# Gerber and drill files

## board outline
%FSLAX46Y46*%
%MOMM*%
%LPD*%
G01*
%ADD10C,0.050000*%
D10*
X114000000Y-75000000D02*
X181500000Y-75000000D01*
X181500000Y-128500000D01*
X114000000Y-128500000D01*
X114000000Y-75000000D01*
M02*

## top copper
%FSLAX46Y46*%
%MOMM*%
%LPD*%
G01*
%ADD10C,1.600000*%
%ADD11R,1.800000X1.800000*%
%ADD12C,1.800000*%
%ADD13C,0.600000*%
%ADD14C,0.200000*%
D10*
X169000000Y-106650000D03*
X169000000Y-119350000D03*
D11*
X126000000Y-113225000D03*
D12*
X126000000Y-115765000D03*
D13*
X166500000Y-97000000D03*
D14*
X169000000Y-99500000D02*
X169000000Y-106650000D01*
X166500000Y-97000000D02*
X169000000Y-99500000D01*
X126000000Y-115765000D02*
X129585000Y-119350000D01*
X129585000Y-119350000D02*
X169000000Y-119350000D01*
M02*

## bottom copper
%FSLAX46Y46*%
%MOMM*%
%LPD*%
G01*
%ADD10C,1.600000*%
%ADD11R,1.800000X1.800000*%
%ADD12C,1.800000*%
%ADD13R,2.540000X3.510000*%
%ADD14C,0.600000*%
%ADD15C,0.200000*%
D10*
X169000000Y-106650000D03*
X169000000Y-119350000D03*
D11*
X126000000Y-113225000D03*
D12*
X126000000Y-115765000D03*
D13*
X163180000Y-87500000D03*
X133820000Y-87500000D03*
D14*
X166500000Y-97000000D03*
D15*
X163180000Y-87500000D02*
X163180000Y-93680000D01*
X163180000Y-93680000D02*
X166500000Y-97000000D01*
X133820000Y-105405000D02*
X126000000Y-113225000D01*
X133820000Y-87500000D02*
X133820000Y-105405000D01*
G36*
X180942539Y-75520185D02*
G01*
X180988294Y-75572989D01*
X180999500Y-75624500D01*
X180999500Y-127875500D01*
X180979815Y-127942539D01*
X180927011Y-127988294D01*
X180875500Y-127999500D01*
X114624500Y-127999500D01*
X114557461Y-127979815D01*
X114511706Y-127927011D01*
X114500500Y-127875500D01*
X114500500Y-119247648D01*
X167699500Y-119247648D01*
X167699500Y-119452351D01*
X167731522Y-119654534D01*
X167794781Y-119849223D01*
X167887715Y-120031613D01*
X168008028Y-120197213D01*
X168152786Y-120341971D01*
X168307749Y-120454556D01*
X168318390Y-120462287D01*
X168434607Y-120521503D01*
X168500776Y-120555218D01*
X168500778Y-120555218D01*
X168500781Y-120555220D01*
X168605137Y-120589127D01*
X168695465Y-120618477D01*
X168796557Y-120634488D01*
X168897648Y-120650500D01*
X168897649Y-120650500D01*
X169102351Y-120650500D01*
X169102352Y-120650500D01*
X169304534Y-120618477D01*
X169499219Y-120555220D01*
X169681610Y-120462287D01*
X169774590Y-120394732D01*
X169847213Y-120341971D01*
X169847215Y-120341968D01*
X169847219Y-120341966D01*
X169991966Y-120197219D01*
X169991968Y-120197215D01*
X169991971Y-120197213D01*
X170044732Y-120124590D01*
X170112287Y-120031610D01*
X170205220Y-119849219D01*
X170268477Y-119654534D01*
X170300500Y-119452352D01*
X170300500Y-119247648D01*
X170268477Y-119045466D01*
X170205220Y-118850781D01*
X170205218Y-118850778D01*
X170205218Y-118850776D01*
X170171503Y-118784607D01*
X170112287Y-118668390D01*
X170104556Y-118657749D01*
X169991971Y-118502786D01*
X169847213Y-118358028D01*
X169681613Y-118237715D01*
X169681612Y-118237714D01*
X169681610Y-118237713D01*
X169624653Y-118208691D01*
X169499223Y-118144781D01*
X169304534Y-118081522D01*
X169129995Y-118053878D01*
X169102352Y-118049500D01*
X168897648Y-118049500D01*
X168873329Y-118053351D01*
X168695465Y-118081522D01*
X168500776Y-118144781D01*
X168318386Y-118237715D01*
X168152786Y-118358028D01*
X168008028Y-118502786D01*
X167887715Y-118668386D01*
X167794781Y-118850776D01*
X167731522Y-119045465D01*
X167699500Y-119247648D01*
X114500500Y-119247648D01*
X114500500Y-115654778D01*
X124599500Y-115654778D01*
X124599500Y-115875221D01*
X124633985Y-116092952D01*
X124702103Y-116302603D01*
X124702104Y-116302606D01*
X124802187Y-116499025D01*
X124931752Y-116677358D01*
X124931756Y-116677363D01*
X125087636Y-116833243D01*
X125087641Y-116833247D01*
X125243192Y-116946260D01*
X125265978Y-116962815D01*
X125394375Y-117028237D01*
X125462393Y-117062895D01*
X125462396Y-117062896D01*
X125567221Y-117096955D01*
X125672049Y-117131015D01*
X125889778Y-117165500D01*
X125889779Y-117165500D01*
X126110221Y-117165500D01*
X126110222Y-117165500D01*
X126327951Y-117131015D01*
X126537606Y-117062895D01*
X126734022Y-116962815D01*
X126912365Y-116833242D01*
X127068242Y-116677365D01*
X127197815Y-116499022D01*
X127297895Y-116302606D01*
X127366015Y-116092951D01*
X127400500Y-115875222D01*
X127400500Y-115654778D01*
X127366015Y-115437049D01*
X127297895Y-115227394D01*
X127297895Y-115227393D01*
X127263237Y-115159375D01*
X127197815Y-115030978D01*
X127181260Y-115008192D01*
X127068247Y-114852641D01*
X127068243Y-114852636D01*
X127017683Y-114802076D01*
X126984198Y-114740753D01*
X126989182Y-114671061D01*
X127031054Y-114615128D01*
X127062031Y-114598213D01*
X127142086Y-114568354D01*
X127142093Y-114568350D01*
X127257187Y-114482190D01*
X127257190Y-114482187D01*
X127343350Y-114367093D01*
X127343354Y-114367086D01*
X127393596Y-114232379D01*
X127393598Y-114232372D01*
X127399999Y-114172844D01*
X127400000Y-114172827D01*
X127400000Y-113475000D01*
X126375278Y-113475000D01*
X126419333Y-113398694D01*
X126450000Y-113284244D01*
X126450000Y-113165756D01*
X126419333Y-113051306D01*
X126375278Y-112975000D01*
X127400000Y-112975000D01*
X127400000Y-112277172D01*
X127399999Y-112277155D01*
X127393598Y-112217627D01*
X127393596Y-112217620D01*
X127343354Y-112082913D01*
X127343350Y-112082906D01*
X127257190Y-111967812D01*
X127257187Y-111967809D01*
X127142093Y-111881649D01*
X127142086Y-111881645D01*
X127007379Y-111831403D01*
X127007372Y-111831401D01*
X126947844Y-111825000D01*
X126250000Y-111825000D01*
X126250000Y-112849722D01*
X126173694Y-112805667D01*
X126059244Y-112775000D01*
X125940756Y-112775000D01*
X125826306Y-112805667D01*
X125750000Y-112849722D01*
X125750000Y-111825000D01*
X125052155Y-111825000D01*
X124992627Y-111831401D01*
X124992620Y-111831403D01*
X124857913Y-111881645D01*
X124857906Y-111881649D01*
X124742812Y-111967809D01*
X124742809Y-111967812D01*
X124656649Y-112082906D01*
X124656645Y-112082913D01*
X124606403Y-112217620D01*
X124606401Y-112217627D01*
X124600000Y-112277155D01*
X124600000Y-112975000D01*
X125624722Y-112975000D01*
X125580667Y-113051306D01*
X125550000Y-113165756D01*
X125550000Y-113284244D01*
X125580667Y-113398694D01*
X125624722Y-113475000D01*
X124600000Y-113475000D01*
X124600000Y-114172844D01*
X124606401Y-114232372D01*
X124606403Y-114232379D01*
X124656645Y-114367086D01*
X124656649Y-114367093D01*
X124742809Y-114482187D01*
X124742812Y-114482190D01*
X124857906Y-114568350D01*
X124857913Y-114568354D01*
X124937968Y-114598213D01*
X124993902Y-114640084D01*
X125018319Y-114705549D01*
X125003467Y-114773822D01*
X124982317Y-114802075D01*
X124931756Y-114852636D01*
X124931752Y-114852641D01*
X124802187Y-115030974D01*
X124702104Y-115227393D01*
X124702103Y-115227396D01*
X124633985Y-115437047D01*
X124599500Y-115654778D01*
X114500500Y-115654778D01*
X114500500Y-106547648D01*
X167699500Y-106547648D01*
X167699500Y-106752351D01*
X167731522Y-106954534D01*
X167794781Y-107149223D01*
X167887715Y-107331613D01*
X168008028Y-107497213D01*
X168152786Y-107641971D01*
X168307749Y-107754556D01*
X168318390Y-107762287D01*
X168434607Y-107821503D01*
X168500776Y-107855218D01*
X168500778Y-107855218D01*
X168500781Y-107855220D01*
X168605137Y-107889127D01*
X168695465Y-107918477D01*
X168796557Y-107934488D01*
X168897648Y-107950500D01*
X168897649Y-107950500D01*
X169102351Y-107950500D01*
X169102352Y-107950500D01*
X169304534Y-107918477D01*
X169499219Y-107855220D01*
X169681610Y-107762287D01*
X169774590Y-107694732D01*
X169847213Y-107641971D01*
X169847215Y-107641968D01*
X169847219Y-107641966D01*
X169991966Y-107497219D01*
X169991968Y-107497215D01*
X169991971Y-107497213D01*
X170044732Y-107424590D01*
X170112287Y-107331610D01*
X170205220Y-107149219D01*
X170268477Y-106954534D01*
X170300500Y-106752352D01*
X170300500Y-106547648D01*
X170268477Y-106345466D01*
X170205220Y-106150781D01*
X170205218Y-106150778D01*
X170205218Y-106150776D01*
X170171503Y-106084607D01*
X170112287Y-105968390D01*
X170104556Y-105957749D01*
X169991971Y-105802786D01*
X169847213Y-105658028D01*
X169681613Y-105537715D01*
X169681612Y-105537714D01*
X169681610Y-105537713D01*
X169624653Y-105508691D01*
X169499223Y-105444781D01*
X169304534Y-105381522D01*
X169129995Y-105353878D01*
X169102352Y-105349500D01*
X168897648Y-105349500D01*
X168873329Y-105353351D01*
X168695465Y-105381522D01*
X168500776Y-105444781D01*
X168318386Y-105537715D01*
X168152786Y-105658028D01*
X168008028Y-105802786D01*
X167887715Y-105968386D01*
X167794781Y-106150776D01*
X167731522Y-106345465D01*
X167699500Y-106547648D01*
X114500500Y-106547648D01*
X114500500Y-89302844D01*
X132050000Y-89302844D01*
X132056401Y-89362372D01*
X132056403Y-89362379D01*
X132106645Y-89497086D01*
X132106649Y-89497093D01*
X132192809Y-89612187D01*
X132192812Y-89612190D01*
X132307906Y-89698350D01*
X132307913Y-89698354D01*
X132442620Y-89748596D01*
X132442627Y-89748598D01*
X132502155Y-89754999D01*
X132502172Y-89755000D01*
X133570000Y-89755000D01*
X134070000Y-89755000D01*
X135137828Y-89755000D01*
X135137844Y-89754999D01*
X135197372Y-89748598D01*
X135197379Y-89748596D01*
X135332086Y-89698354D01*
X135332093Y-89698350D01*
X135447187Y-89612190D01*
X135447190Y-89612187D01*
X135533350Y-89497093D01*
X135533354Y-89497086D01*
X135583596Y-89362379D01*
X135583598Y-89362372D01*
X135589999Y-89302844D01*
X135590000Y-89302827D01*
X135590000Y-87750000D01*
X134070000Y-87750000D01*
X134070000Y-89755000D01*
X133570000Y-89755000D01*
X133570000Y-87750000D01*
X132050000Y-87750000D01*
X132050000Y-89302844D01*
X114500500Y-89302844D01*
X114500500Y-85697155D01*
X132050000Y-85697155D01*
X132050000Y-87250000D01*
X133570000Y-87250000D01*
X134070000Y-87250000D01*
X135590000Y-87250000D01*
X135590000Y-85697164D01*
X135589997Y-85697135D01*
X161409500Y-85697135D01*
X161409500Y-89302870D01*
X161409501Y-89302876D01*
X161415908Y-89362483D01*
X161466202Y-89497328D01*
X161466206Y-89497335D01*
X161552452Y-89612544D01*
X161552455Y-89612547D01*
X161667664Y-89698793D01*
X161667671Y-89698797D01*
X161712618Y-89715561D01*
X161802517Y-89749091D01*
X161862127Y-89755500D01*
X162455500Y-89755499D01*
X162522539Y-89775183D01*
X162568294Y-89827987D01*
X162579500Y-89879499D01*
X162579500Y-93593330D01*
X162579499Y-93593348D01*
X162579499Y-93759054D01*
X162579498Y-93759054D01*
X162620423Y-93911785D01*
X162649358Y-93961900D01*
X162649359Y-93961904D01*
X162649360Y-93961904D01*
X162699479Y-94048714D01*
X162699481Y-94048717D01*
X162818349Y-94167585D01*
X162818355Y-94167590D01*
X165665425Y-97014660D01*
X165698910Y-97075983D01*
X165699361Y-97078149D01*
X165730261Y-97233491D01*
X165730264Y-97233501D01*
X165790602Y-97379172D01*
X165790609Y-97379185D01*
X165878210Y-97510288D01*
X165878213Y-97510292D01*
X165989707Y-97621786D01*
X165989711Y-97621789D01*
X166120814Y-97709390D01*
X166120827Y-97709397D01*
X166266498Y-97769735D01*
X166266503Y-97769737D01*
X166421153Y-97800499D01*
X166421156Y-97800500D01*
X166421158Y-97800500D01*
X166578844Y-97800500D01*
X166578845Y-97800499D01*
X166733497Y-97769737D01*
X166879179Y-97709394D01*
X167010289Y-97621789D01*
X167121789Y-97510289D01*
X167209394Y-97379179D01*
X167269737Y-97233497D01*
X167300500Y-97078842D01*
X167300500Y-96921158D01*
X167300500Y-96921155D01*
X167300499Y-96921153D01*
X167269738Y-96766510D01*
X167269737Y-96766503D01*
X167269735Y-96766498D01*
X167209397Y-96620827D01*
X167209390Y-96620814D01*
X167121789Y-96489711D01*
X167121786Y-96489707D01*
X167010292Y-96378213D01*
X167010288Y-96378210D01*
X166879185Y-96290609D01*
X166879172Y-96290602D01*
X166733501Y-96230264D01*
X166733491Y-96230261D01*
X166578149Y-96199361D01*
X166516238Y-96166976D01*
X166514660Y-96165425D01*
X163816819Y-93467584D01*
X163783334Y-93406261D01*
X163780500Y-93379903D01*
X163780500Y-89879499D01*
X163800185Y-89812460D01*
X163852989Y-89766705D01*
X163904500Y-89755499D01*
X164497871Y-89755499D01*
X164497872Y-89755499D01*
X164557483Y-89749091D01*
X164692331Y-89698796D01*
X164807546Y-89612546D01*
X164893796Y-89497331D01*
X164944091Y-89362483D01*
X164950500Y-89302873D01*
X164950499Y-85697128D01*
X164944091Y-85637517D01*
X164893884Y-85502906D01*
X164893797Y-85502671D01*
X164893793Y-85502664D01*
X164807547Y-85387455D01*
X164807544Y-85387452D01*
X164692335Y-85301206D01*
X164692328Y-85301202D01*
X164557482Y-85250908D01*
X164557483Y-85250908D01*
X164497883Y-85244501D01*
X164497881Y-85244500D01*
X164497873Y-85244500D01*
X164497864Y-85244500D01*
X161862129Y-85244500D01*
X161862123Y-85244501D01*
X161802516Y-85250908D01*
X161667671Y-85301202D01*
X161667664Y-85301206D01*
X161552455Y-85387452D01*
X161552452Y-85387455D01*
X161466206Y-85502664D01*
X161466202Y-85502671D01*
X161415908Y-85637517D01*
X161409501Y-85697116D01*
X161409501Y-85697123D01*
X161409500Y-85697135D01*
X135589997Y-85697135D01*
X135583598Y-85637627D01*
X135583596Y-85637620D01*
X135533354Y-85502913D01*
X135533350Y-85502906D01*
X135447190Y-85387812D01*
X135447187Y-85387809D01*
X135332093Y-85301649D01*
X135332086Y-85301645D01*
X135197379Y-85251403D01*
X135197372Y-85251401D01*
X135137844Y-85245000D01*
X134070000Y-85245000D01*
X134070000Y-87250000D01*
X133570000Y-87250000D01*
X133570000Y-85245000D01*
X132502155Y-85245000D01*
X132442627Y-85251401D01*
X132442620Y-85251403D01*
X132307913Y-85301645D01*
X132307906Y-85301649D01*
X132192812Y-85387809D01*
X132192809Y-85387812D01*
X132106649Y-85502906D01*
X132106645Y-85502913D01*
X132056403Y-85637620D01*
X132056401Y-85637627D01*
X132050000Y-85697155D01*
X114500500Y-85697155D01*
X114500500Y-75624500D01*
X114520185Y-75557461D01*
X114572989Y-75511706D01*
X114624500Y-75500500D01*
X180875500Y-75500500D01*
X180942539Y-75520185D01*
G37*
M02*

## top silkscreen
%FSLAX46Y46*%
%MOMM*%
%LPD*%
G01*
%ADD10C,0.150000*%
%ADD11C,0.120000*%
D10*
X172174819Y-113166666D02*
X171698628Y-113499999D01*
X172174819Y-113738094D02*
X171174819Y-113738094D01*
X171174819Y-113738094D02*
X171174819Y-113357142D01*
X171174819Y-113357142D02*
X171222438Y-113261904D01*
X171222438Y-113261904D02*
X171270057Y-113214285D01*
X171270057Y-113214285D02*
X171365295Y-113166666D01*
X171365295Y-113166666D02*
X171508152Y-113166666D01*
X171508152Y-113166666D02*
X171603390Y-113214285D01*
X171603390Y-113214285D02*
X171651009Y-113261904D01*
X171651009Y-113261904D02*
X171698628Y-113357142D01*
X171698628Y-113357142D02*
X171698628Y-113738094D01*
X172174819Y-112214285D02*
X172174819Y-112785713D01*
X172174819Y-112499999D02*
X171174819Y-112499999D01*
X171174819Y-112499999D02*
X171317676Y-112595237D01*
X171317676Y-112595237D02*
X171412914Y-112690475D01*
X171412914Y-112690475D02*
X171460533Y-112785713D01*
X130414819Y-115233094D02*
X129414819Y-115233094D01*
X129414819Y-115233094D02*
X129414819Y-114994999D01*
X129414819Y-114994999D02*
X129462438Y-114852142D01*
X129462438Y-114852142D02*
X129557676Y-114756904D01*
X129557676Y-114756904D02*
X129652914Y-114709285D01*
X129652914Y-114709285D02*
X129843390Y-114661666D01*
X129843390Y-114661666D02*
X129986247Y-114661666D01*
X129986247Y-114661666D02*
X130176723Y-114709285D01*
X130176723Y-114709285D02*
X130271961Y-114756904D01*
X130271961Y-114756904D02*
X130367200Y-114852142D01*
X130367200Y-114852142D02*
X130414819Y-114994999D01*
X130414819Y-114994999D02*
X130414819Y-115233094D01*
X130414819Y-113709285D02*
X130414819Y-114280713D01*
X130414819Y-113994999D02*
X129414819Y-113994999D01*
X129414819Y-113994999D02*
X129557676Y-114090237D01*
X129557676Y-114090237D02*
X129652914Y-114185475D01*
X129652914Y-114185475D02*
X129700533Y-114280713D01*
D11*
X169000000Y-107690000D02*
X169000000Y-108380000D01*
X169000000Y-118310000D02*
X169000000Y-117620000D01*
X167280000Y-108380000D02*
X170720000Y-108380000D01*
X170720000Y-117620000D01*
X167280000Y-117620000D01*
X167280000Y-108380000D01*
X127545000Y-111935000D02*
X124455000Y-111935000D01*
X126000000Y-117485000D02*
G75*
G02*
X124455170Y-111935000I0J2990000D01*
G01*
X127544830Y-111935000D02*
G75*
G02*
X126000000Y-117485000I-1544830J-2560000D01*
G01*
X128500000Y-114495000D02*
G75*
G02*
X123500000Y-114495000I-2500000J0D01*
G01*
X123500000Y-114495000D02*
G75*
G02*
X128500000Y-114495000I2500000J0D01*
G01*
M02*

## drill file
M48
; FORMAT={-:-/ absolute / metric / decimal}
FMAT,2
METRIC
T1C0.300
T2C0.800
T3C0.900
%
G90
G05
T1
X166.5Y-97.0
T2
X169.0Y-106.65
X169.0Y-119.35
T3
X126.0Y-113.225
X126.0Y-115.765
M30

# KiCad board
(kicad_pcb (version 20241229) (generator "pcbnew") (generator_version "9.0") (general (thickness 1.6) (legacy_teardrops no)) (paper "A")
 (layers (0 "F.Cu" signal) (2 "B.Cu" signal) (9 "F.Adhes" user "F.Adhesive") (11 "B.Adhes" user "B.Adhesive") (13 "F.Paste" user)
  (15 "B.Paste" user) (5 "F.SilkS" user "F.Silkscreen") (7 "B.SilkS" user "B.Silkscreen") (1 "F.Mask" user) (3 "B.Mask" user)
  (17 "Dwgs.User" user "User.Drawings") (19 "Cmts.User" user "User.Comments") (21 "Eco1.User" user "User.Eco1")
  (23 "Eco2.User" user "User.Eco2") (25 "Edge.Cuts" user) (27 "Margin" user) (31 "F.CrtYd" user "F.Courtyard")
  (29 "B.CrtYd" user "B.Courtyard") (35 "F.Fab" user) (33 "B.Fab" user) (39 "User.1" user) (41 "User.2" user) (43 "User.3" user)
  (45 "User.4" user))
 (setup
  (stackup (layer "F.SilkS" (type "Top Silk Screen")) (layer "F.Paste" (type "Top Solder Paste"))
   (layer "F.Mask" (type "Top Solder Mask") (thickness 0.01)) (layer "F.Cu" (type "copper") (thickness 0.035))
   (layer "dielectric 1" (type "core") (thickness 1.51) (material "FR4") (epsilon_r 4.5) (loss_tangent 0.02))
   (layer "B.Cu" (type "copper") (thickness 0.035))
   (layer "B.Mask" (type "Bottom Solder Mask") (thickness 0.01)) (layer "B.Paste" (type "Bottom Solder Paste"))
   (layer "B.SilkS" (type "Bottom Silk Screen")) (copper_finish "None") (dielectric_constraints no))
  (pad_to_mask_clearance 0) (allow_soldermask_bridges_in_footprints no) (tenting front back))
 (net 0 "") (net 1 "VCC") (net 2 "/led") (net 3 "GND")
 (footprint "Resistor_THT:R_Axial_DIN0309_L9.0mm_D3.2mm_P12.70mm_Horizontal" (layer "F.Cu") (at 169 106.65 -90)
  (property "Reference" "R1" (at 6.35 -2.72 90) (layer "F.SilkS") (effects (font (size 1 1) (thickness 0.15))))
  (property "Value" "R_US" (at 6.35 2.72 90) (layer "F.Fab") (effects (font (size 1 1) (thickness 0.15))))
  (fp_line (start 1.04 0) (end 1.73 0) (stroke (width 0.12) (type solid)) (layer "F.SilkS"))
  (fp_line (start 11.66 0) (end 10.97 0) (stroke (width 0.12) (type solid)) (layer "F.SilkS"))
  (fp_rect (start 1.73 -1.72) (end 10.97 1.72) (stroke (width 0.12) (type solid)) (fill no) (layer "F.SilkS"))
  (pad "1" thru_hole circle (at 0 0 270) (size 1.6 1.6) (drill 0.8) (layers "*.Cu" "*.Mask") (remove_unused_layers no) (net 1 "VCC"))
  (pad "2" thru_hole circle (at 12.7 0 270) (size 1.6 1.6) (drill 0.8) (layers "*.Cu" "*.Mask") (remove_unused_layers no) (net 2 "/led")))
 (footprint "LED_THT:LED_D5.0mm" (layer "F.Cu") (at 126 113.225 -90)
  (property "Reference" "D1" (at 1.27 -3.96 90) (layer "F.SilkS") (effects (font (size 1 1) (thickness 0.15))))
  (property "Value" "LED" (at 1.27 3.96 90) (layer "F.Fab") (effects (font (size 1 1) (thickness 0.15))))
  (fp_line (start -1.29 -1.545) (end -1.29 1.545) (stroke (width 0.12) (type solid)) (layer "F.SilkS"))
  (fp_arc (start 4.26 0) (mid 2.071779 2.880495) (end -1.29 1.54483) (stroke (width 0.12) (type solid)) (layer "F.SilkS"))
  (fp_arc (start -1.29 -1.54483) (mid 2.071779 -2.880495) (end 4.26 0) (stroke (width 0.12) (type solid)) (layer "F.SilkS"))
  (fp_circle (center 1.27 0) (end 3.77 0) (stroke (width 0.12) (type solid)) (fill no) (layer "F.SilkS"))
  (pad "1" thru_hole rect (at 0 0 270) (size 1.8 1.8) (drill 0.9) (layers "*.Cu" "*.Mask") (remove_unused_layers no) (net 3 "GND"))
  (pad "2" thru_hole circle (at 2.54 0 270) (size 1.8 1.8) (drill 0.9) (layers "*.Cu" "*.Mask") (remove_unused_layers no) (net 2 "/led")))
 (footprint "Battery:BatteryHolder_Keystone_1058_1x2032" (layer "B.Cu") (at 148.5 87.5 180)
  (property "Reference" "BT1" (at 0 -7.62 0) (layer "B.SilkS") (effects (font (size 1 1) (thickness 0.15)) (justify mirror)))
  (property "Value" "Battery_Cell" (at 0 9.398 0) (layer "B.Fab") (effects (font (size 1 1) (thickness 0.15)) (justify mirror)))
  (pad "1" smd rect (at -14.68 0 180) (size 2.54 3.51) (layers "B.Cu" "B.Mask" "B.Paste") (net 1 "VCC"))
  (pad "2" smd rect (at 14.68 0 180) (size 2.54 3.51) (layers "B.Cu" "B.Mask" "B.Paste") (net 3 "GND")))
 (gr_rect (start 114 75) (end 181.5 128.5) (stroke (width 0.05) (type default)) (fill no) (layer "Edge.Cuts"))
 (segment (start 169 99.5) (end 169 106.65) (width 0.2) (layer "F.Cu") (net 1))
 (segment (start 166.5 97) (end 169 99.5) (width 0.2) (layer "F.Cu") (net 1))
 (via (at 166.5 97) (size 0.6) (drill 0.3) (layers "F.Cu" "B.Cu") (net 1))
 (segment (start 163.18 87.5) (end 163.18 93.68) (width 0.2) (layer "B.Cu") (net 1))
 (segment (start 163.18 93.68) (end 166.5 97) (width 0.2) (layer "B.Cu") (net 1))
 (segment (start 133.82 105.405) (end 126 113.225) (width 0.2) (layer "B.Cu") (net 3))
 (segment (start 133.82 87.5) (end 133.82 105.405) (width 0.2) (layer "B.Cu") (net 3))
 (segment (start 126 115.765) (end 129.585 119.35) (width 0.2) (layer "F.Cu") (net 2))
 (segment (start 129.585 119.35) (end 169 119.35) (width 0.2) (layer "F.Cu") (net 2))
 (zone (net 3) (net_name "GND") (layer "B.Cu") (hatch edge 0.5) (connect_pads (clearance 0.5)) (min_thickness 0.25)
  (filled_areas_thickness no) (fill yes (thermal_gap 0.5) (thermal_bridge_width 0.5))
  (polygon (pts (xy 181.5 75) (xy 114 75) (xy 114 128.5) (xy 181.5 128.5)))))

